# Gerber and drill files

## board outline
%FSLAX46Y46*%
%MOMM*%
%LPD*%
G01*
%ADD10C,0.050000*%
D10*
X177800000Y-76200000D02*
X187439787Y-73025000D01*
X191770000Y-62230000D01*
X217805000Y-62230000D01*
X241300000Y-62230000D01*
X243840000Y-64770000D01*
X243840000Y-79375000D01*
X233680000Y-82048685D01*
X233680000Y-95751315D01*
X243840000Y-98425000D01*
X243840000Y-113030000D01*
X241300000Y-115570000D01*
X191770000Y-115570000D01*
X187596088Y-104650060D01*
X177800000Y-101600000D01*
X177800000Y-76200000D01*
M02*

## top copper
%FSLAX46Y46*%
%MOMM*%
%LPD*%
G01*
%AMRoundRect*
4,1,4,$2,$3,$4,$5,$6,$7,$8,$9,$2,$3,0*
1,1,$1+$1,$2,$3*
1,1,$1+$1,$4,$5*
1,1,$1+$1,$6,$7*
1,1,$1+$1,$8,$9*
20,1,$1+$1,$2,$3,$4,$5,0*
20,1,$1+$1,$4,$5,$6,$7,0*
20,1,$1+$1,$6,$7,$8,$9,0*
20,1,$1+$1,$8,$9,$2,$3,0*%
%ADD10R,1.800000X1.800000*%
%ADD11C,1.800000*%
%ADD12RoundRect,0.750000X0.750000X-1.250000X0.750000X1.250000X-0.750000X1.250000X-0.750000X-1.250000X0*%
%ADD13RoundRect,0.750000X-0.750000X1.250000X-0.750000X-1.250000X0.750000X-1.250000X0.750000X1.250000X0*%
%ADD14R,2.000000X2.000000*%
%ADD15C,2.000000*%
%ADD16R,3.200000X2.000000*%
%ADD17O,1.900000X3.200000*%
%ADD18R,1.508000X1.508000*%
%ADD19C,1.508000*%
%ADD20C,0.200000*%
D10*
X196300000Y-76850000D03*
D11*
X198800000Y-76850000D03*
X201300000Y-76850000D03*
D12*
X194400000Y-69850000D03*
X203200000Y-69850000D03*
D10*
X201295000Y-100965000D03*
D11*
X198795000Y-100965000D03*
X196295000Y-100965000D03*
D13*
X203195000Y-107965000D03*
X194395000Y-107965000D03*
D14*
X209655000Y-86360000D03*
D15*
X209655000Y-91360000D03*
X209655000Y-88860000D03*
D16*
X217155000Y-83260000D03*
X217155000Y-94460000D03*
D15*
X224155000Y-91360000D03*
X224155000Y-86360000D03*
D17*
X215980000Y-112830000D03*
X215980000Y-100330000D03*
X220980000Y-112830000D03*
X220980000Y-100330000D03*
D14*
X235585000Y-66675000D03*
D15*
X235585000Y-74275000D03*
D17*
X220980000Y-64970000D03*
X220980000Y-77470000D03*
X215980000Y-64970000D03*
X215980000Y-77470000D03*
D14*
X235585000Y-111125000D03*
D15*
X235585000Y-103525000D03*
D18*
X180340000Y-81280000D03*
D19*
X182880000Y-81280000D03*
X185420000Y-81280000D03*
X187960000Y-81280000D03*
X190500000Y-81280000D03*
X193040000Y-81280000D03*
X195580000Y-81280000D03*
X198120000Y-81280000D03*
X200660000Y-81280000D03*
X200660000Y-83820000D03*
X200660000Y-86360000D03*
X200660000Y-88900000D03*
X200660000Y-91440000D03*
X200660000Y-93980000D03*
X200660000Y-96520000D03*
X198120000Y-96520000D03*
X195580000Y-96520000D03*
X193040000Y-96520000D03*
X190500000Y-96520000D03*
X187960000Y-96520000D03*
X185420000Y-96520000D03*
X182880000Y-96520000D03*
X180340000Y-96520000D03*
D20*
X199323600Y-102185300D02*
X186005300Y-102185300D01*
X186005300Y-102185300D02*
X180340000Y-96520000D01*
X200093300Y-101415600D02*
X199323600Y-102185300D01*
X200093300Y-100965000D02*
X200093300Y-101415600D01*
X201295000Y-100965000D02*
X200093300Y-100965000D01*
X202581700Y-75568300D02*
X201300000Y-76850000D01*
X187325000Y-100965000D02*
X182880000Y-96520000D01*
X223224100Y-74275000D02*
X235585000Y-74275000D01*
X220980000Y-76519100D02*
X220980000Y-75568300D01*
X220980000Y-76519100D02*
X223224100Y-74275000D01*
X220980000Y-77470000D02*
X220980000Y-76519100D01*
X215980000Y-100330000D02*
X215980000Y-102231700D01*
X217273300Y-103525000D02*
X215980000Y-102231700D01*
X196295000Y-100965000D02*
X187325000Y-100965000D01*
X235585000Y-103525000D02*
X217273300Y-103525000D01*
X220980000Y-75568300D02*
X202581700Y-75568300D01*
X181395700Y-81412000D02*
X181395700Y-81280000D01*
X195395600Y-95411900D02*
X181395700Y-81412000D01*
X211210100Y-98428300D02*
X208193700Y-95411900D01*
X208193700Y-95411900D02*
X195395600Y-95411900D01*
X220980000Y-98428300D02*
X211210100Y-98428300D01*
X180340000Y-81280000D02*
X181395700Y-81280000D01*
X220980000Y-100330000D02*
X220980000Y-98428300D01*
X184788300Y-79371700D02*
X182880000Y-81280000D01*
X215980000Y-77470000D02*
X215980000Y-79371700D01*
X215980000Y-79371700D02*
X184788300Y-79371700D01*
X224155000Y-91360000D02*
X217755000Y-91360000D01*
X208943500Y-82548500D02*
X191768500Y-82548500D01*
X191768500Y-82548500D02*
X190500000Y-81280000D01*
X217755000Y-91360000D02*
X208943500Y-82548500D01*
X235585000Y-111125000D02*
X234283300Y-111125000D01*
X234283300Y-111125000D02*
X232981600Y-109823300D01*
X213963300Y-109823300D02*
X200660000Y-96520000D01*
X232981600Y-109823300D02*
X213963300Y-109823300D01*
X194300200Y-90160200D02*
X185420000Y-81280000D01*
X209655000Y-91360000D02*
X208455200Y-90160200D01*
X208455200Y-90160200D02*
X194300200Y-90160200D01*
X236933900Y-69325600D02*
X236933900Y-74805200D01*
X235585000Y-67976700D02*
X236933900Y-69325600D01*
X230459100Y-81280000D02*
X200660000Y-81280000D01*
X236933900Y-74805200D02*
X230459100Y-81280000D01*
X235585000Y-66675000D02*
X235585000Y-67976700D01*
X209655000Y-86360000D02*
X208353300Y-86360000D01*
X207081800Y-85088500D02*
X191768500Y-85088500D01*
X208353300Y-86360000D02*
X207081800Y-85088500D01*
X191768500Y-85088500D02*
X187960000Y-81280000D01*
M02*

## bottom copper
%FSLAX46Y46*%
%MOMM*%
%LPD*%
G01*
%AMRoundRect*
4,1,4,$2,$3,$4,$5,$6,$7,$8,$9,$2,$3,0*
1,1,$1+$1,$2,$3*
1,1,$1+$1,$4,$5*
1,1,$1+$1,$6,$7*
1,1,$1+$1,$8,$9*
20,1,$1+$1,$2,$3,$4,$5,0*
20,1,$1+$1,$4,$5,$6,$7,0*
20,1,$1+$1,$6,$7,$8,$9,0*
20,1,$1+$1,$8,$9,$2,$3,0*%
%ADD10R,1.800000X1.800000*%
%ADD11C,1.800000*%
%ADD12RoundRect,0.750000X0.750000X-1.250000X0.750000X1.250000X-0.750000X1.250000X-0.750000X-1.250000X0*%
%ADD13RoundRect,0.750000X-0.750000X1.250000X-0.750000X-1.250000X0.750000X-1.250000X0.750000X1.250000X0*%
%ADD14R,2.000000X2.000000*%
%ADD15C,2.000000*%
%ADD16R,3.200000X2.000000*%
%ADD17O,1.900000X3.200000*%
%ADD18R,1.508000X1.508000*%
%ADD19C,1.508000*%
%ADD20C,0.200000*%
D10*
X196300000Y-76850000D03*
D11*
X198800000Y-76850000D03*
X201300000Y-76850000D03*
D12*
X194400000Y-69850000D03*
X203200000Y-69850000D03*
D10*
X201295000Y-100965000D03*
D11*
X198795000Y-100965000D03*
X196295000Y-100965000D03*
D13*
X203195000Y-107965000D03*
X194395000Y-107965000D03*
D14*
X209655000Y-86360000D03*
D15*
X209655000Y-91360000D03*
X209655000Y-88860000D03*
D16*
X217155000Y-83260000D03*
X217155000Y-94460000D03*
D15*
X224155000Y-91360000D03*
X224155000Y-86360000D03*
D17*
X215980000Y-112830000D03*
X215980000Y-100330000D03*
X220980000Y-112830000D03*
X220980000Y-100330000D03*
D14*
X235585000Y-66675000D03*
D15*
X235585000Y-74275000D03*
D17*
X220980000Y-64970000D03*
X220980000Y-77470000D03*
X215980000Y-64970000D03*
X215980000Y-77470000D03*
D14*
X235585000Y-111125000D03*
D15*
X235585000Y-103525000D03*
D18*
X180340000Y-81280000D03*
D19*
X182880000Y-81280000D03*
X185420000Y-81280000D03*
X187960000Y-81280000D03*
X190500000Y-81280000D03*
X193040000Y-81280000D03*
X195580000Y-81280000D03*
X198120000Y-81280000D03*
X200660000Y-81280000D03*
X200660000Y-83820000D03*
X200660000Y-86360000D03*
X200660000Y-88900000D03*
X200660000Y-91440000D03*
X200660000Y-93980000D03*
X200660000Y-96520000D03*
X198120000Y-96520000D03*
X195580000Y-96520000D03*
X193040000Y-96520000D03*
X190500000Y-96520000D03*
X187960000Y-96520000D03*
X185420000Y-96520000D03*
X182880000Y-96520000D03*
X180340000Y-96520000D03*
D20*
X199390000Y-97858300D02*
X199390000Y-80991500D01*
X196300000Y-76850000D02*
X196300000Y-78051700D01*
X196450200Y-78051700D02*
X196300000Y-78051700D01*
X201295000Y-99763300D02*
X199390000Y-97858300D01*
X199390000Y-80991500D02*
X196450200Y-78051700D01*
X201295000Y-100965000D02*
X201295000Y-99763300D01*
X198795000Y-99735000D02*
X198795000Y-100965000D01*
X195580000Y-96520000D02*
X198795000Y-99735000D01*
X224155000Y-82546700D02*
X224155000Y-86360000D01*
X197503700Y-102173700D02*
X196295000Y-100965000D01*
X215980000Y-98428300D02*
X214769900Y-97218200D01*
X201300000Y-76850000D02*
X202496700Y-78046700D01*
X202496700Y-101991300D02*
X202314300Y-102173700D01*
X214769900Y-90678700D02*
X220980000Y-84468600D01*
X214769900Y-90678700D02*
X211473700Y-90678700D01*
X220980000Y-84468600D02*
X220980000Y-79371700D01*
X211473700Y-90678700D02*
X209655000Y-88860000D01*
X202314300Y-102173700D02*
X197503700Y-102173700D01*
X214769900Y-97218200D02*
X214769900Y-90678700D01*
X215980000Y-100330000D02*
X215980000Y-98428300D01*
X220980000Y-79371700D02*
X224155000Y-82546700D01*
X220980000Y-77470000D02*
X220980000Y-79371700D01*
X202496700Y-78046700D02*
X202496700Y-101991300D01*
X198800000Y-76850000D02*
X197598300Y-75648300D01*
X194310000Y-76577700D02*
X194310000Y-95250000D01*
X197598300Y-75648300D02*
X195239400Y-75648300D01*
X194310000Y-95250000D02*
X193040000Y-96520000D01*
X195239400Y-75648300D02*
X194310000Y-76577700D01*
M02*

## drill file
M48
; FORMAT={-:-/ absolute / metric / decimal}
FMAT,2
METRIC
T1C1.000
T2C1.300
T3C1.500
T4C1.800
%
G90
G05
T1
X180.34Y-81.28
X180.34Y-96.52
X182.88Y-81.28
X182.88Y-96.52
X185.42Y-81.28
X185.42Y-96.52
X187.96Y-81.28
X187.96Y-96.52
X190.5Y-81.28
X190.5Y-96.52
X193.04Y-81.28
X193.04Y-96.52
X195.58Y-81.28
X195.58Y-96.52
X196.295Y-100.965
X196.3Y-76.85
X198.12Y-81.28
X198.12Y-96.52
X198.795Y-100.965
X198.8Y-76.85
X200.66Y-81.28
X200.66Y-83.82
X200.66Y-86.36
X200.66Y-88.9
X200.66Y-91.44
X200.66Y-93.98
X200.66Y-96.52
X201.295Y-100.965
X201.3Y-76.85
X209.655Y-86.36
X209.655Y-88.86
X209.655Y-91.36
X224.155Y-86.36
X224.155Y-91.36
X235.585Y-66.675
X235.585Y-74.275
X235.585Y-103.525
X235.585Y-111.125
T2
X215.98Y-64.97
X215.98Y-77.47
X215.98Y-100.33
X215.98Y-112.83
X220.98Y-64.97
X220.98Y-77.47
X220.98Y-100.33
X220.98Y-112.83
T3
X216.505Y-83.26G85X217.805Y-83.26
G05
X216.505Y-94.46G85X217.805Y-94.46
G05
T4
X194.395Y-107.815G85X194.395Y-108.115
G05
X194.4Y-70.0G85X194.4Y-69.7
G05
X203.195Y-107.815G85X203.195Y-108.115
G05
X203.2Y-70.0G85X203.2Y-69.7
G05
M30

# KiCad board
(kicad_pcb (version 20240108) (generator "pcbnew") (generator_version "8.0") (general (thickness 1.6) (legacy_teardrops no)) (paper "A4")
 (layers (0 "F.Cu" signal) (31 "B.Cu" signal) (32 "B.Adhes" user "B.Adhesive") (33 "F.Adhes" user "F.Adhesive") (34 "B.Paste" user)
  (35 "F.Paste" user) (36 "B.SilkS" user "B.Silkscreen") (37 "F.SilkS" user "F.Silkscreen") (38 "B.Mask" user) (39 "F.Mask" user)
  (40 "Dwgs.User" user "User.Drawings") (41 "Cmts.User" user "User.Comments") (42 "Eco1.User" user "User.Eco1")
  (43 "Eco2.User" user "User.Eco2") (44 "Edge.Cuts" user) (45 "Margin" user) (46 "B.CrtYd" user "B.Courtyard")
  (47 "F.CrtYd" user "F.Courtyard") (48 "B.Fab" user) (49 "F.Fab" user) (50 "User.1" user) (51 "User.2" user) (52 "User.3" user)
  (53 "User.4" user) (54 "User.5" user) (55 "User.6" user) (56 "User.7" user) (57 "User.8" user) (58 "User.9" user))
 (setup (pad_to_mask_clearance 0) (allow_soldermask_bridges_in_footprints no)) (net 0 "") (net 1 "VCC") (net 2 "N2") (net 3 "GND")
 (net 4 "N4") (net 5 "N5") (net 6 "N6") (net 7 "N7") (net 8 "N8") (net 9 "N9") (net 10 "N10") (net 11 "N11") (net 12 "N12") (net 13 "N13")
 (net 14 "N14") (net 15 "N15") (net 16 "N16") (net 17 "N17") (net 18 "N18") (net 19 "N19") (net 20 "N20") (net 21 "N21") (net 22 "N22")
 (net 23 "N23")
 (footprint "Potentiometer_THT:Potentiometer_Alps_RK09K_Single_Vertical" (layer "F.Cu") (at 196.3 76.85 90)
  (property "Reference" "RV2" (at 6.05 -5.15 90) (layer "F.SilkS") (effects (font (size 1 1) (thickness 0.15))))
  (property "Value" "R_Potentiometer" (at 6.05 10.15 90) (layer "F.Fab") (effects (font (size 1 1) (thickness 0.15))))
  (pad "1" thru_hole rect (at 0 0 90) (size 1.8 1.8) (drill 1) (layers "*.Cu" "*.Mask") (remove_unused_layers no) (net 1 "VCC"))
  (pad "2" thru_hole circle (at 0 2.5 90) (size 1.8 1.8) (drill 1) (layers "*.Cu" "*.Mask") (remove_unused_layers no) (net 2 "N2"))
  (pad "3" thru_hole circle (at 0 5 90) (size 1.8 1.8) (drill 1) (layers "*.Cu" "*.Mask") (remove_unused_layers no) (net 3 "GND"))
  (pad "MP" thru_hole roundrect (at 7 -1.9 90) (size 4 3) (drill oval 2.1 1.8) (layers "*.Cu" "*.Mask") (remove_unused_layers no)
   (roundrect_rratio 0.25))
  (pad "MP" thru_hole roundrect (at 7 6.9 90) (size 4 3) (drill oval 2.1 1.8) (layers "*.Cu" "*.Mask") (remove_unused_layers no)
   (roundrect_rratio 0.25)))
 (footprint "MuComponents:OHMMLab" (layer "F.Cu") (at 227.33 88.9 90)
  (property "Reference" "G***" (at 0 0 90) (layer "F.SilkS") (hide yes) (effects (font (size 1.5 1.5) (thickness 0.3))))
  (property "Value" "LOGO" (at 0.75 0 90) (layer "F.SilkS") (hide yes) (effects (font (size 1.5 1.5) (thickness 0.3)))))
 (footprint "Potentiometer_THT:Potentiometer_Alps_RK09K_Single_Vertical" (layer "F.Cu") (at 201.295 100.965 -90)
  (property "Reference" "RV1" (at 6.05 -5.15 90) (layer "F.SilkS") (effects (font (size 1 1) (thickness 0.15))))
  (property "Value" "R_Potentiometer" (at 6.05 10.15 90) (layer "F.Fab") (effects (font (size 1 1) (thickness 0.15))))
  (pad "1" thru_hole rect (at 0 0 270) (size 1.8 1.8) (drill 1) (layers "*.Cu" "*.Mask") (remove_unused_layers no) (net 1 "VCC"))
  (pad "2" thru_hole circle (at 0 2.5 270) (size 1.8 1.8) (drill 1) (layers "*.Cu" "*.Mask") (remove_unused_layers no) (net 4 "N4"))
  (pad "3" thru_hole circle (at 0 5 270) (size 1.8 1.8) (drill 1) (layers "*.Cu" "*.Mask") (remove_unused_layers no) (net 3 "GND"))
  (pad "MP" thru_hole roundrect (at 7 -1.9 270) (size 4 3) (drill oval 2.1 1.8) (layers "*.Cu" "*.Mask") (remove_unused_layers no)
   (roundrect_rratio 0.25))
  (pad "MP" thru_hole roundrect (at 7 6.9 270) (size 4 3) (drill oval 2.1 1.8) (layers "*.Cu" "*.Mask") (remove_unused_layers no)
   (roundrect_rratio 0.25)))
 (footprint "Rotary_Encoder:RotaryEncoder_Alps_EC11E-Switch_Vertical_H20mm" (layer "F.Cu") (at 209.655 86.36)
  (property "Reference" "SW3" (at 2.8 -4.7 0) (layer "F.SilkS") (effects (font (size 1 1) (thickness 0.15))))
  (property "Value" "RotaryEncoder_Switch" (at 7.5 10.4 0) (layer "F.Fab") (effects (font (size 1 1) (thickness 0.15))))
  (pad "A" thru_hole rect (at 0 0) (size 2 2) (drill 1) (layers "*.Cu" "*.Mask") (remove_unused_layers no) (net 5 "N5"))
  (pad "B" thru_hole circle (at 0 5) (size 2 2) (drill 1) (layers "*.Cu" "*.Mask") (remove_unused_layers no) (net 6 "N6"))
  (pad "C" thru_hole circle (at 0 2.5) (size 2 2) (drill 1) (layers "*.Cu" "*.Mask") (remove_unused_layers no) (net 3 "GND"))
  (pad "MP" thru_hole rect (at 7.5 -3.1) (size 3.2 2) (drill oval 2.8 1.5) (layers "*.Cu" "*.Mask") (remove_unused_layers no))
  (pad "MP" thru_hole rect (at 7.5 8.1) (size 3.2 2) (drill oval 2.8 1.5) (layers "*.Cu" "*.Mask") (remove_unused_layers no))
  (pad "S1" thru_hole circle (at 14.5 5) (size 2 2) (drill 1) (layers "*.Cu" "*.Mask") (remove_unused_layers no) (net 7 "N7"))
  (pad "S2" thru_hole circle (at 14.5 0) (size 2 2) (drill 1) (layers "*.Cu" "*.Mask") (remove_unused_layers no) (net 3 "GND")))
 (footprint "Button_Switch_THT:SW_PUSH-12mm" (layer "F.Cu") (at 215.98 112.83 90)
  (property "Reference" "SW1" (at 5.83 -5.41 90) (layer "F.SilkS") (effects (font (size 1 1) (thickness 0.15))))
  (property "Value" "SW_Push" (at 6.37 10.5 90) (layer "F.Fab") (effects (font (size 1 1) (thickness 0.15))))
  (pad "1" thru_hole oval (at 0 0 90) (size 3.2 1.9) (drill 1.3) (layers "*.Cu" "*.Mask") (remove_unused_layers no))
  (pad "1" thru_hole oval (at 12.5 0 90) (size 3.2 1.9) (drill 1.3) (layers "*.Cu" "*.Mask") (remove_unused_layers no) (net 3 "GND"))
  (pad "2" thru_hole oval (at 0 5 90) (size 3.2 1.9) (drill 1.3) (layers "*.Cu" "*.Mask") (remove_unused_layers no))
  (pad "2" thru_hole oval (at 12.5 5 90) (size 3.2 1.9) (drill 1.3) (layers "*.Cu" "*.Mask") (remove_unused_layers no) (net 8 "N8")))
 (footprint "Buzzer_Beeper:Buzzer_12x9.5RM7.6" (layer "F.Cu") (at 235.585 66.675 -90)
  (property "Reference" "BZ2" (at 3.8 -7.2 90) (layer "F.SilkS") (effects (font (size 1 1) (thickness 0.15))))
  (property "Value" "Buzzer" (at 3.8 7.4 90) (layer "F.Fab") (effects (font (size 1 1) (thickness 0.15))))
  (pad "1" thru_hole rect (at 0 0 270) (size 2 2) (drill 1) (layers "*.Cu" "*.Mask") (remove_unused_layers no) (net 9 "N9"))
  (pad "2" thru_hole circle (at 7.6 0 270) (size 2 2) (drill 1) (layers "*.Cu" "*.Mask") (remove_unused_layers no) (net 3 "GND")))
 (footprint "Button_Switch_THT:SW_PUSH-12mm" (layer "F.Cu") (at 220.98 64.97 -90)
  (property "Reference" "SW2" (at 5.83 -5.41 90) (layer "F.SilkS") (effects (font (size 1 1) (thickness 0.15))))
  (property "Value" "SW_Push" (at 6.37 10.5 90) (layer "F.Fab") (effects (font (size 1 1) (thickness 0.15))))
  (pad "1" thru_hole oval (at 0 0 270) (size 3.2 1.9) (drill 1.3) (layers "*.Cu" "*.Mask") (remove_unused_layers no))
  (pad "1" thru_hole oval (at 12.5 0 270) (size 3.2 1.9) (drill 1.3) (layers "*.Cu" "*.Mask") (remove_unused_layers no) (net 3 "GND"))
  (pad "2" thru_hole oval (at 0 5 270) (size 3.2 1.9) (drill 1.3) (layers "*.Cu" "*.Mask") (remove_unused_layers no))
  (pad "2" thru_hole oval (at 12.5 5 270) (size 3.2 1.9) (drill 1.3) (layers "*.Cu" "*.Mask") (remove_unused_layers no) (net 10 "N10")))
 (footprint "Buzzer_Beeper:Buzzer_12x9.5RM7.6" (layer "F.Cu") (at 235.585 111.125 90)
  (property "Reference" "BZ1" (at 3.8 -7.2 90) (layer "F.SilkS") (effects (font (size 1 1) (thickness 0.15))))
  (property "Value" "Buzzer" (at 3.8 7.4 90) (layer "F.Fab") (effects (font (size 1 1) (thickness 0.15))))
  (pad "1" thru_hole rect (at 0 0 90) (size 2 2) (drill 1) (layers "*.Cu" "*.Mask") (remove_unused_layers no) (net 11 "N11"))
  (pad "2" thru_hole circle (at 7.6 0 90) (size 2 2) (drill 1) (layers "*.Cu" "*.Mask") (remove_unused_layers no) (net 3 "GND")))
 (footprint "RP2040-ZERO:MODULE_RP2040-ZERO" (layer "F.Cu") (at 190.5 88.9 90)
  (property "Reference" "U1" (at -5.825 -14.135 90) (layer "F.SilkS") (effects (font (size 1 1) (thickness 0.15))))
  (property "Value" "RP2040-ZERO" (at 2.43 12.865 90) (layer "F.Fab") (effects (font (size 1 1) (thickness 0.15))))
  (pad "1" thru_hole rect (at 7.62 -10.16 90) (size 1.508 1.508) (drill 1) (layers "*.Cu" "*.Mask") (remove_unused_layers no) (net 8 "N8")
   (solder_mask_margin 0.102))
  (pad "2" thru_hole circle (at 7.62 -7.62 90) (size 1.508 1.508) (drill 1) (layers "*.Cu" "*.Mask") (remove_unused_layers no)
   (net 10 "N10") (solder_mask_margin 0.102))
  (pad "3" thru_hole circle (at 7.62 -5.08 90) (size 1.508 1.508) (drill 1) (layers "*.Cu" "*.Mask") (remove_unused_layers no) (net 6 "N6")
   (solder_mask_margin 0.102))
  (pad "4" thru_hole circle (at 7.62 -2.54 90) (size 1.508 1.508) (drill 1) (layers "*.Cu" "*.Mask") (remove_unused_layers no) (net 5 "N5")
   (solder_mask_margin 0.102))
  (pad "5" thru_hole circle (at 7.62 0 90) (size 1.508 1.508) (drill 1) (layers "*.Cu" "*.Mask") (remove_unused_layers no) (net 7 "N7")
   (solder_mask_margin 0.102))
  (pad "6" thru_hole circle (at 7.62 2.54 90) (size 1.508 1.508) (drill 1) (layers "*.Cu" "*.Mask") (remove_unused_layers no) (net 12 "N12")
   (solder_mask_margin 0.102))
  (pad "7" thru_hole circle (at 7.62 5.08 90) (size 1.508 1.508) (drill 1) (layers "*.Cu" "*.Mask") (remove_unused_layers no) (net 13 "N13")
   (solder_mask_margin 0.102))
  (pad "8" thru_hole circle (at 7.62 7.62 90) (size 1.508 1.508) (drill 1) (layers "*.Cu" "*.Mask") (remove_unused_layers no) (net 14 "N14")
   (solder_mask_margin 0.102))
  (pad "9" thru_hole circle (at 7.62 10.16 90) (size 1.508 1.508) (drill 1) (layers "*.Cu" "*.Mask") (remove_unused_layers no) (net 9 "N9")
   (solder_mask_margin 0.102))
  (pad "10" thru_hole circle (at 5.08 10.16 90) (size 1.508 1.508) (drill 1) (layers "*.Cu" "*.Mask") (remove_unused_layers no)
   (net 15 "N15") (solder_mask_margin 0.102))
  (pad "11" thru_hole circle (at 2.54 10.16 90) (size 1.508 1.508) (drill 1) (layers "*.Cu" "*.Mask") (remove_unused_layers no)
   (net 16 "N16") (solder_mask_margin 0.102))
  (pad "12" thru_hole circle (at 0 10.16 90) (size 1.508 1.508) (drill 1) (layers "*.Cu" "*.Mask") (remove_unused_layers no) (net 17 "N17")
   (solder_mask_margin 0.102))
  (pad "13" thru_hole circle (at -2.54 10.16 90) (size 1.508 1.508) (drill 1) (layers "*.Cu" "*.Mask") (remove_unused_layers no)
   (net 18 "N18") (solder_mask_margin 0.102))
  (pad "14" thru_hole circle (at -5.08 10.16 90) (size 1.508 1.508) (drill 1) (layers "*.Cu" "*.Mask") (remove_unused_layers no)
   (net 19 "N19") (solder_mask_margin 0.102))
  (pad "15" thru_hole circle (at -7.62 10.16 90) (size 1.508 1.508) (drill 1) (layers "*.Cu" "*.Mask") (remove_unused_layers no)
   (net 11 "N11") (solder_mask_margin 0.102))
  (pad "16" thru_hole circle (at -7.62 7.62 90) (size 1.508 1.508) (drill 1) (layers "*.Cu" "*.Mask") (remove_unused_layers no)
   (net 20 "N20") (solder_mask_margin 0.102))
  (pad "17" thru_hole circle (at -7.62 5.08 90) (size 1.508 1.508) (drill 1) (layers "*.Cu" "*.Mask") (remove_unused_layers no) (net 4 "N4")
   (solder_mask_margin 0.102))
  (pad "18" thru_hole circle (at -7.62 2.54 90) (size 1.508 1.508) (drill 1) (layers "*.Cu" "*.Mask") (remove_unused_layers no) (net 2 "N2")
   (solder_mask_margin 0.102))
  (pad "19" thru_hole circle (at -7.62 0 90) (size 1.508 1.508) (drill 1) (layers "*.Cu" "*.Mask") (remove_unused_layers no) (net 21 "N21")
   (solder_mask_margin 0.102))
  (pad "20" thru_hole circle (at -7.62 -2.54 90) (size 1.508 1.508) (drill 1) (layers "*.Cu" "*.Mask") (remove_unused_layers no)
   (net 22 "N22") (solder_mask_margin 0.102))
  (pad "21" thru_hole circle (at -7.62 -5.08 90) (size 1.508 1.508) (drill 1) (layers "*.Cu" "*.Mask") (remove_unused_layers no)
   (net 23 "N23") (solder_mask_margin 0.102))
  (pad "22" thru_hole circle (at -7.62 -7.62 90) (size 1.508 1.508) (drill 1) (layers "*.Cu" "*.Mask") (remove_unused_layers no)
   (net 3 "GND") (solder_mask_margin 0.102))
  (pad "23" thru_hole circle (at -7.62 -10.16 90) (size 1.508 1.508) (drill 1) (layers "*.Cu" "*.Mask") (remove_unused_layers no)
   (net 1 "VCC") (solder_mask_margin 0.102)))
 (gr_poly
  (pts (xy 177.8 76.2) (xy 187.439787 73.025) (xy 191.77 62.23) (xy 217.805 62.23) (xy 241.3 62.23) (xy 243.84 64.77) (xy 243.84 79.375)
   (xy 233.68 82.048685) (xy 233.68 95.751315) (xy 243.84 98.425) (xy 243.84 113.03) (xy 241.3 115.57) (xy 191.77 115.57)
   (xy 187.596088 104.65006) (xy 177.8 101.6))
  (stroke (width 0.05) (type solid)) (fill none) (layer "Edge.Cuts"))
 (segment (start 199.3236 102.1853) (end 186.0053 102.1853) (width 0.2) (layer "F.Cu") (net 1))
 (segment (start 186.0053 102.1853) (end 180.34 96.52) (width 0.2) (layer "F.Cu") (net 1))
 (segment (start 200.0933 101.4156) (end 199.3236 102.1853) (width 0.2) (layer "F.Cu") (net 1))
 (segment (start 200.0933 100.965) (end 200.0933 101.4156) (width 0.2) (layer "F.Cu") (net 1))
 (segment (start 201.295 100.965) (end 200.0933 100.965) (width 0.2) (layer "F.Cu") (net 1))
 (segment (start 199.39 97.8583) (end 199.39 80.9915) (width 0.2) (layer "B.Cu") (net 1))
 (segment (start 196.3 76.85) (end 196.3 78.0517) (width 0.2) (layer "B.Cu") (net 1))
 (segment (start 196.4502 78.0517) (end 196.3 78.0517) (width 0.2) (layer "B.Cu") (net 1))
 (segment (start 201.295 99.7633) (end 199.39 97.8583) (width 0.2) (layer "B.Cu") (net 1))
 (segment (start 199.39 80.9915) (end 196.4502 78.0517) (width 0.2) (layer "B.Cu") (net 1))
 (segment (start 201.295 100.965) (end 201.295 99.7633) (width 0.2) (layer "B.Cu") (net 1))
 (segment (start 198.795 99.735) (end 198.795 100.965) (width 0.2) (layer "B.Cu") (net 4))
 (segment (start 195.58 96.52) (end 198.795 99.735) (width 0.2) (layer "B.Cu") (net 4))
 (segment (start 202.5817 75.5683) (end 201.3 76.85) (width 0.2) (layer "F.Cu") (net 3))
 (segment (start 187.325 100.965) (end 182.88 96.52) (width 0.2) (layer "F.Cu") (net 3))
 (segment (start 223.2241 74.275) (end 235.585 74.275) (width 0.2) (layer "F.Cu") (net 3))
 (segment (start 220.98 76.5191) (end 220.98 75.5683) (width 0.2) (layer "F.Cu") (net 3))
 (segment (start 220.98 76.5191) (end 223.2241 74.275) (width 0.2) (layer "F.Cu") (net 3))
 (segment (start 220.98 77.47) (end 220.98 76.5191) (width 0.2) (layer "F.Cu") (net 3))
 (segment (start 215.98 100.33) (end 215.98 102.2317) (width 0.2) (layer "F.Cu") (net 3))
 (segment (start 217.2733 103.525) (end 215.98 102.2317) (width 0.2) (layer "F.Cu") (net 3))
 (segment (start 196.295 100.965) (end 187.325 100.965) (width 0.2) (layer "F.Cu") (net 3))
 (segment (start 235.585 103.525) (end 217.2733 103.525) (width 0.2) (layer "F.Cu") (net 3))
 (segment (start 220.98 75.5683) (end 202.5817 75.5683) (width 0.2) (layer "F.Cu") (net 3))
 (segment (start 224.155 82.5467) (end 224.155 86.36) (width 0.2) (layer "B.Cu") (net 3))
 (segment (start 197.5037 102.1737) (end 196.295 100.965) (width 0.2) (layer "B.Cu") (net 3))
 (segment (start 215.98 98.4283) (end 214.7699 97.2182) (width 0.2) (layer "B.Cu") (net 3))
 (segment (start 201.3 76.85) (end 202.4967 78.0467) (width 0.2) (layer "B.Cu") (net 3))
 (segment (start 202.4967 101.9913) (end 202.3143 102.1737) (width 0.2) (layer "B.Cu") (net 3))
 (segment (start 214.7699 90.6787) (end 220.98 84.4686) (width 0.2) (layer "B.Cu") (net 3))
 (segment (start 214.7699 90.6787) (end 211.4737 90.6787) (width 0.2) (layer "B.Cu") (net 3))
 (segment (start 220.98 84.4686) (end 220.98 79.3717) (width 0.2) (layer "B.Cu") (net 3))
 (segment (start 211.4737 90.6787) (end 209.655 88.86) (width 0.2) (layer "B.Cu") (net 3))
 (segment (start 202.3143 102.1737) (end 197.5037 102.1737) (width 0.2) (layer "B.Cu") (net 3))
 (segment (start 214.7699 97.2182) (end 214.7699 90.6787) (width 0.2) (layer "B.Cu") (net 3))
 (segment (start 215.98 100.33) (end 215.98 98.4283) (width 0.2) (layer "B.Cu") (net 3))
 (segment (start 220.98 79.3717) (end 224.155 82.5467) (width 0.2) (layer "B.Cu") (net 3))
 (segment (start 220.98 77.47) (end 220.98 79.3717) (width 0.2) (layer "B.Cu") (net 3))
 (segment (start 202.4967 78.0467) (end 202.4967 101.9913) (width 0.2) (layer "B.Cu") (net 3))
 (segment (start 198.8 76.85) (end 197.5983 75.6483) (width 0.2) (layer "B.Cu") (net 2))
 (segment (start 194.31 76.5777) (end 194.31 95.25) (width 0.2) (layer "B.Cu") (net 2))
 (segment (start 197.5983 75.6483) (end 195.2394 75.6483) (width 0.2) (layer "B.Cu") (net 2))
 (segment (start 194.31 95.25) (end 193.04 96.52) (width 0.2) (layer "B.Cu") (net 2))
 (segment (start 195.2394 75.6483) (end 194.31 76.5777) (width 0.2) (layer "B.Cu") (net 2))
 (segment (start 181.3957 81.412) (end 181.3957 81.28) (width 0.2) (layer "F.Cu") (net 8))
 (segment (start 195.3956 95.4119) (end 181.3957 81.412) (width 0.2) (layer "F.Cu") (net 8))
 (segment (start 211.2101 98.4283) (end 208.1937 95.4119) (width 0.2) (layer "F.Cu") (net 8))
 (segment (start 208.1937 95.4119) (end 195.3956 95.4119) (width 0.2) (layer "F.Cu") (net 8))
 (segment (start 220.98 98.4283) (end 211.2101 98.4283) (width 0.2) (layer "F.Cu") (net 8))
 (segment (start 180.34 81.28) (end 181.3957 81.28) (width 0.2) (layer "F.Cu") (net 8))
 (segment (start 220.98 100.33) (end 220.98 98.4283) (width 0.2) (layer "F.Cu") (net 8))
 (segment (start 184.7883 79.3717) (end 182.88 81.28) (width 0.2) (layer "F.Cu") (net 10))
 (segment (start 215.98 77.47) (end 215.98 79.3717) (width 0.2) (layer "F.Cu") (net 10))
 (segment (start 215.98 79.3717) (end 184.7883 79.3717) (width 0.2) (layer "F.Cu") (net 10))
 (segment (start 224.155 91.36) (end 217.755 91.36) (width 0.2) (layer "F.Cu") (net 7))
 (segment (start 208.9435 82.5485) (end 191.7685 82.5485) (width 0.2) (layer "F.Cu") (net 7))
 (segment (start 191.7685 82.5485) (end 190.5 81.28) (width 0.2) (layer "F.Cu") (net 7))
 (segment (start 217.755 91.36) (end 208.9435 82.5485) (width 0.2) (layer "F.Cu") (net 7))
 (segment (start 235.585 111.125) (end 234.2833 111.125) (width 0.2) (layer "F.Cu") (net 11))
 (segment (start 234.2833 111.125) (end 232.9816 109.8233) (width 0.2) (layer "F.Cu") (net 11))
 (segment (start 213.9633 109.8233) (end 200.66 96.52) (width 0.2) (layer "F.Cu") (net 11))
 (segment (start 232.9816 109.8233) (end 213.9633 109.8233) (width 0.2) (layer "F.Cu") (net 11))
 (segment (start 194.3002 90.1602) (end 185.42 81.28) (width 0.2) (layer "F.Cu") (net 6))
 (segment (start 209.655 91.36) (end 208.4552 90.1602) (width 0.2) (layer "F.Cu") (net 6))
 (segment (start 208.4552 90.1602) (end 194.3002 90.1602) (width 0.2) (layer "F.Cu") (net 6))
 (segment (start 236.9339 69.3256) (end 236.9339 74.8052) (width 0.2) (layer "F.Cu") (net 9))
 (segment (start 235.585 67.9767) (end 236.9339 69.3256) (width 0.2) (layer "F.Cu") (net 9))
 (segment (start 230.4591 81.28) (end 200.66 81.28) (width 0.2) (layer "F.Cu") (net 9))
 (segment (start 236.9339 74.8052) (end 230.4591 81.28) (width 0.2) (layer "F.Cu") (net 9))
 (segment (start 235.585 66.675) (end 235.585 67.9767) (width 0.2) (layer "F.Cu") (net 9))
 (segment (start 209.655 86.36) (end 208.3533 86.36) (width 0.2) (layer "F.Cu") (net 5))
 (segment (start 207.0818 85.0885) (end 191.7685 85.0885) (width 0.2) (layer "F.Cu") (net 5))
 (segment (start 208.3533 86.36) (end 207.0818 85.0885) (width 0.2) (layer "F.Cu") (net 5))
 (segment (start 191.7685 85.0885) (end 187.96 81.28) (width 0.2) (layer "F.Cu") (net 5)))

